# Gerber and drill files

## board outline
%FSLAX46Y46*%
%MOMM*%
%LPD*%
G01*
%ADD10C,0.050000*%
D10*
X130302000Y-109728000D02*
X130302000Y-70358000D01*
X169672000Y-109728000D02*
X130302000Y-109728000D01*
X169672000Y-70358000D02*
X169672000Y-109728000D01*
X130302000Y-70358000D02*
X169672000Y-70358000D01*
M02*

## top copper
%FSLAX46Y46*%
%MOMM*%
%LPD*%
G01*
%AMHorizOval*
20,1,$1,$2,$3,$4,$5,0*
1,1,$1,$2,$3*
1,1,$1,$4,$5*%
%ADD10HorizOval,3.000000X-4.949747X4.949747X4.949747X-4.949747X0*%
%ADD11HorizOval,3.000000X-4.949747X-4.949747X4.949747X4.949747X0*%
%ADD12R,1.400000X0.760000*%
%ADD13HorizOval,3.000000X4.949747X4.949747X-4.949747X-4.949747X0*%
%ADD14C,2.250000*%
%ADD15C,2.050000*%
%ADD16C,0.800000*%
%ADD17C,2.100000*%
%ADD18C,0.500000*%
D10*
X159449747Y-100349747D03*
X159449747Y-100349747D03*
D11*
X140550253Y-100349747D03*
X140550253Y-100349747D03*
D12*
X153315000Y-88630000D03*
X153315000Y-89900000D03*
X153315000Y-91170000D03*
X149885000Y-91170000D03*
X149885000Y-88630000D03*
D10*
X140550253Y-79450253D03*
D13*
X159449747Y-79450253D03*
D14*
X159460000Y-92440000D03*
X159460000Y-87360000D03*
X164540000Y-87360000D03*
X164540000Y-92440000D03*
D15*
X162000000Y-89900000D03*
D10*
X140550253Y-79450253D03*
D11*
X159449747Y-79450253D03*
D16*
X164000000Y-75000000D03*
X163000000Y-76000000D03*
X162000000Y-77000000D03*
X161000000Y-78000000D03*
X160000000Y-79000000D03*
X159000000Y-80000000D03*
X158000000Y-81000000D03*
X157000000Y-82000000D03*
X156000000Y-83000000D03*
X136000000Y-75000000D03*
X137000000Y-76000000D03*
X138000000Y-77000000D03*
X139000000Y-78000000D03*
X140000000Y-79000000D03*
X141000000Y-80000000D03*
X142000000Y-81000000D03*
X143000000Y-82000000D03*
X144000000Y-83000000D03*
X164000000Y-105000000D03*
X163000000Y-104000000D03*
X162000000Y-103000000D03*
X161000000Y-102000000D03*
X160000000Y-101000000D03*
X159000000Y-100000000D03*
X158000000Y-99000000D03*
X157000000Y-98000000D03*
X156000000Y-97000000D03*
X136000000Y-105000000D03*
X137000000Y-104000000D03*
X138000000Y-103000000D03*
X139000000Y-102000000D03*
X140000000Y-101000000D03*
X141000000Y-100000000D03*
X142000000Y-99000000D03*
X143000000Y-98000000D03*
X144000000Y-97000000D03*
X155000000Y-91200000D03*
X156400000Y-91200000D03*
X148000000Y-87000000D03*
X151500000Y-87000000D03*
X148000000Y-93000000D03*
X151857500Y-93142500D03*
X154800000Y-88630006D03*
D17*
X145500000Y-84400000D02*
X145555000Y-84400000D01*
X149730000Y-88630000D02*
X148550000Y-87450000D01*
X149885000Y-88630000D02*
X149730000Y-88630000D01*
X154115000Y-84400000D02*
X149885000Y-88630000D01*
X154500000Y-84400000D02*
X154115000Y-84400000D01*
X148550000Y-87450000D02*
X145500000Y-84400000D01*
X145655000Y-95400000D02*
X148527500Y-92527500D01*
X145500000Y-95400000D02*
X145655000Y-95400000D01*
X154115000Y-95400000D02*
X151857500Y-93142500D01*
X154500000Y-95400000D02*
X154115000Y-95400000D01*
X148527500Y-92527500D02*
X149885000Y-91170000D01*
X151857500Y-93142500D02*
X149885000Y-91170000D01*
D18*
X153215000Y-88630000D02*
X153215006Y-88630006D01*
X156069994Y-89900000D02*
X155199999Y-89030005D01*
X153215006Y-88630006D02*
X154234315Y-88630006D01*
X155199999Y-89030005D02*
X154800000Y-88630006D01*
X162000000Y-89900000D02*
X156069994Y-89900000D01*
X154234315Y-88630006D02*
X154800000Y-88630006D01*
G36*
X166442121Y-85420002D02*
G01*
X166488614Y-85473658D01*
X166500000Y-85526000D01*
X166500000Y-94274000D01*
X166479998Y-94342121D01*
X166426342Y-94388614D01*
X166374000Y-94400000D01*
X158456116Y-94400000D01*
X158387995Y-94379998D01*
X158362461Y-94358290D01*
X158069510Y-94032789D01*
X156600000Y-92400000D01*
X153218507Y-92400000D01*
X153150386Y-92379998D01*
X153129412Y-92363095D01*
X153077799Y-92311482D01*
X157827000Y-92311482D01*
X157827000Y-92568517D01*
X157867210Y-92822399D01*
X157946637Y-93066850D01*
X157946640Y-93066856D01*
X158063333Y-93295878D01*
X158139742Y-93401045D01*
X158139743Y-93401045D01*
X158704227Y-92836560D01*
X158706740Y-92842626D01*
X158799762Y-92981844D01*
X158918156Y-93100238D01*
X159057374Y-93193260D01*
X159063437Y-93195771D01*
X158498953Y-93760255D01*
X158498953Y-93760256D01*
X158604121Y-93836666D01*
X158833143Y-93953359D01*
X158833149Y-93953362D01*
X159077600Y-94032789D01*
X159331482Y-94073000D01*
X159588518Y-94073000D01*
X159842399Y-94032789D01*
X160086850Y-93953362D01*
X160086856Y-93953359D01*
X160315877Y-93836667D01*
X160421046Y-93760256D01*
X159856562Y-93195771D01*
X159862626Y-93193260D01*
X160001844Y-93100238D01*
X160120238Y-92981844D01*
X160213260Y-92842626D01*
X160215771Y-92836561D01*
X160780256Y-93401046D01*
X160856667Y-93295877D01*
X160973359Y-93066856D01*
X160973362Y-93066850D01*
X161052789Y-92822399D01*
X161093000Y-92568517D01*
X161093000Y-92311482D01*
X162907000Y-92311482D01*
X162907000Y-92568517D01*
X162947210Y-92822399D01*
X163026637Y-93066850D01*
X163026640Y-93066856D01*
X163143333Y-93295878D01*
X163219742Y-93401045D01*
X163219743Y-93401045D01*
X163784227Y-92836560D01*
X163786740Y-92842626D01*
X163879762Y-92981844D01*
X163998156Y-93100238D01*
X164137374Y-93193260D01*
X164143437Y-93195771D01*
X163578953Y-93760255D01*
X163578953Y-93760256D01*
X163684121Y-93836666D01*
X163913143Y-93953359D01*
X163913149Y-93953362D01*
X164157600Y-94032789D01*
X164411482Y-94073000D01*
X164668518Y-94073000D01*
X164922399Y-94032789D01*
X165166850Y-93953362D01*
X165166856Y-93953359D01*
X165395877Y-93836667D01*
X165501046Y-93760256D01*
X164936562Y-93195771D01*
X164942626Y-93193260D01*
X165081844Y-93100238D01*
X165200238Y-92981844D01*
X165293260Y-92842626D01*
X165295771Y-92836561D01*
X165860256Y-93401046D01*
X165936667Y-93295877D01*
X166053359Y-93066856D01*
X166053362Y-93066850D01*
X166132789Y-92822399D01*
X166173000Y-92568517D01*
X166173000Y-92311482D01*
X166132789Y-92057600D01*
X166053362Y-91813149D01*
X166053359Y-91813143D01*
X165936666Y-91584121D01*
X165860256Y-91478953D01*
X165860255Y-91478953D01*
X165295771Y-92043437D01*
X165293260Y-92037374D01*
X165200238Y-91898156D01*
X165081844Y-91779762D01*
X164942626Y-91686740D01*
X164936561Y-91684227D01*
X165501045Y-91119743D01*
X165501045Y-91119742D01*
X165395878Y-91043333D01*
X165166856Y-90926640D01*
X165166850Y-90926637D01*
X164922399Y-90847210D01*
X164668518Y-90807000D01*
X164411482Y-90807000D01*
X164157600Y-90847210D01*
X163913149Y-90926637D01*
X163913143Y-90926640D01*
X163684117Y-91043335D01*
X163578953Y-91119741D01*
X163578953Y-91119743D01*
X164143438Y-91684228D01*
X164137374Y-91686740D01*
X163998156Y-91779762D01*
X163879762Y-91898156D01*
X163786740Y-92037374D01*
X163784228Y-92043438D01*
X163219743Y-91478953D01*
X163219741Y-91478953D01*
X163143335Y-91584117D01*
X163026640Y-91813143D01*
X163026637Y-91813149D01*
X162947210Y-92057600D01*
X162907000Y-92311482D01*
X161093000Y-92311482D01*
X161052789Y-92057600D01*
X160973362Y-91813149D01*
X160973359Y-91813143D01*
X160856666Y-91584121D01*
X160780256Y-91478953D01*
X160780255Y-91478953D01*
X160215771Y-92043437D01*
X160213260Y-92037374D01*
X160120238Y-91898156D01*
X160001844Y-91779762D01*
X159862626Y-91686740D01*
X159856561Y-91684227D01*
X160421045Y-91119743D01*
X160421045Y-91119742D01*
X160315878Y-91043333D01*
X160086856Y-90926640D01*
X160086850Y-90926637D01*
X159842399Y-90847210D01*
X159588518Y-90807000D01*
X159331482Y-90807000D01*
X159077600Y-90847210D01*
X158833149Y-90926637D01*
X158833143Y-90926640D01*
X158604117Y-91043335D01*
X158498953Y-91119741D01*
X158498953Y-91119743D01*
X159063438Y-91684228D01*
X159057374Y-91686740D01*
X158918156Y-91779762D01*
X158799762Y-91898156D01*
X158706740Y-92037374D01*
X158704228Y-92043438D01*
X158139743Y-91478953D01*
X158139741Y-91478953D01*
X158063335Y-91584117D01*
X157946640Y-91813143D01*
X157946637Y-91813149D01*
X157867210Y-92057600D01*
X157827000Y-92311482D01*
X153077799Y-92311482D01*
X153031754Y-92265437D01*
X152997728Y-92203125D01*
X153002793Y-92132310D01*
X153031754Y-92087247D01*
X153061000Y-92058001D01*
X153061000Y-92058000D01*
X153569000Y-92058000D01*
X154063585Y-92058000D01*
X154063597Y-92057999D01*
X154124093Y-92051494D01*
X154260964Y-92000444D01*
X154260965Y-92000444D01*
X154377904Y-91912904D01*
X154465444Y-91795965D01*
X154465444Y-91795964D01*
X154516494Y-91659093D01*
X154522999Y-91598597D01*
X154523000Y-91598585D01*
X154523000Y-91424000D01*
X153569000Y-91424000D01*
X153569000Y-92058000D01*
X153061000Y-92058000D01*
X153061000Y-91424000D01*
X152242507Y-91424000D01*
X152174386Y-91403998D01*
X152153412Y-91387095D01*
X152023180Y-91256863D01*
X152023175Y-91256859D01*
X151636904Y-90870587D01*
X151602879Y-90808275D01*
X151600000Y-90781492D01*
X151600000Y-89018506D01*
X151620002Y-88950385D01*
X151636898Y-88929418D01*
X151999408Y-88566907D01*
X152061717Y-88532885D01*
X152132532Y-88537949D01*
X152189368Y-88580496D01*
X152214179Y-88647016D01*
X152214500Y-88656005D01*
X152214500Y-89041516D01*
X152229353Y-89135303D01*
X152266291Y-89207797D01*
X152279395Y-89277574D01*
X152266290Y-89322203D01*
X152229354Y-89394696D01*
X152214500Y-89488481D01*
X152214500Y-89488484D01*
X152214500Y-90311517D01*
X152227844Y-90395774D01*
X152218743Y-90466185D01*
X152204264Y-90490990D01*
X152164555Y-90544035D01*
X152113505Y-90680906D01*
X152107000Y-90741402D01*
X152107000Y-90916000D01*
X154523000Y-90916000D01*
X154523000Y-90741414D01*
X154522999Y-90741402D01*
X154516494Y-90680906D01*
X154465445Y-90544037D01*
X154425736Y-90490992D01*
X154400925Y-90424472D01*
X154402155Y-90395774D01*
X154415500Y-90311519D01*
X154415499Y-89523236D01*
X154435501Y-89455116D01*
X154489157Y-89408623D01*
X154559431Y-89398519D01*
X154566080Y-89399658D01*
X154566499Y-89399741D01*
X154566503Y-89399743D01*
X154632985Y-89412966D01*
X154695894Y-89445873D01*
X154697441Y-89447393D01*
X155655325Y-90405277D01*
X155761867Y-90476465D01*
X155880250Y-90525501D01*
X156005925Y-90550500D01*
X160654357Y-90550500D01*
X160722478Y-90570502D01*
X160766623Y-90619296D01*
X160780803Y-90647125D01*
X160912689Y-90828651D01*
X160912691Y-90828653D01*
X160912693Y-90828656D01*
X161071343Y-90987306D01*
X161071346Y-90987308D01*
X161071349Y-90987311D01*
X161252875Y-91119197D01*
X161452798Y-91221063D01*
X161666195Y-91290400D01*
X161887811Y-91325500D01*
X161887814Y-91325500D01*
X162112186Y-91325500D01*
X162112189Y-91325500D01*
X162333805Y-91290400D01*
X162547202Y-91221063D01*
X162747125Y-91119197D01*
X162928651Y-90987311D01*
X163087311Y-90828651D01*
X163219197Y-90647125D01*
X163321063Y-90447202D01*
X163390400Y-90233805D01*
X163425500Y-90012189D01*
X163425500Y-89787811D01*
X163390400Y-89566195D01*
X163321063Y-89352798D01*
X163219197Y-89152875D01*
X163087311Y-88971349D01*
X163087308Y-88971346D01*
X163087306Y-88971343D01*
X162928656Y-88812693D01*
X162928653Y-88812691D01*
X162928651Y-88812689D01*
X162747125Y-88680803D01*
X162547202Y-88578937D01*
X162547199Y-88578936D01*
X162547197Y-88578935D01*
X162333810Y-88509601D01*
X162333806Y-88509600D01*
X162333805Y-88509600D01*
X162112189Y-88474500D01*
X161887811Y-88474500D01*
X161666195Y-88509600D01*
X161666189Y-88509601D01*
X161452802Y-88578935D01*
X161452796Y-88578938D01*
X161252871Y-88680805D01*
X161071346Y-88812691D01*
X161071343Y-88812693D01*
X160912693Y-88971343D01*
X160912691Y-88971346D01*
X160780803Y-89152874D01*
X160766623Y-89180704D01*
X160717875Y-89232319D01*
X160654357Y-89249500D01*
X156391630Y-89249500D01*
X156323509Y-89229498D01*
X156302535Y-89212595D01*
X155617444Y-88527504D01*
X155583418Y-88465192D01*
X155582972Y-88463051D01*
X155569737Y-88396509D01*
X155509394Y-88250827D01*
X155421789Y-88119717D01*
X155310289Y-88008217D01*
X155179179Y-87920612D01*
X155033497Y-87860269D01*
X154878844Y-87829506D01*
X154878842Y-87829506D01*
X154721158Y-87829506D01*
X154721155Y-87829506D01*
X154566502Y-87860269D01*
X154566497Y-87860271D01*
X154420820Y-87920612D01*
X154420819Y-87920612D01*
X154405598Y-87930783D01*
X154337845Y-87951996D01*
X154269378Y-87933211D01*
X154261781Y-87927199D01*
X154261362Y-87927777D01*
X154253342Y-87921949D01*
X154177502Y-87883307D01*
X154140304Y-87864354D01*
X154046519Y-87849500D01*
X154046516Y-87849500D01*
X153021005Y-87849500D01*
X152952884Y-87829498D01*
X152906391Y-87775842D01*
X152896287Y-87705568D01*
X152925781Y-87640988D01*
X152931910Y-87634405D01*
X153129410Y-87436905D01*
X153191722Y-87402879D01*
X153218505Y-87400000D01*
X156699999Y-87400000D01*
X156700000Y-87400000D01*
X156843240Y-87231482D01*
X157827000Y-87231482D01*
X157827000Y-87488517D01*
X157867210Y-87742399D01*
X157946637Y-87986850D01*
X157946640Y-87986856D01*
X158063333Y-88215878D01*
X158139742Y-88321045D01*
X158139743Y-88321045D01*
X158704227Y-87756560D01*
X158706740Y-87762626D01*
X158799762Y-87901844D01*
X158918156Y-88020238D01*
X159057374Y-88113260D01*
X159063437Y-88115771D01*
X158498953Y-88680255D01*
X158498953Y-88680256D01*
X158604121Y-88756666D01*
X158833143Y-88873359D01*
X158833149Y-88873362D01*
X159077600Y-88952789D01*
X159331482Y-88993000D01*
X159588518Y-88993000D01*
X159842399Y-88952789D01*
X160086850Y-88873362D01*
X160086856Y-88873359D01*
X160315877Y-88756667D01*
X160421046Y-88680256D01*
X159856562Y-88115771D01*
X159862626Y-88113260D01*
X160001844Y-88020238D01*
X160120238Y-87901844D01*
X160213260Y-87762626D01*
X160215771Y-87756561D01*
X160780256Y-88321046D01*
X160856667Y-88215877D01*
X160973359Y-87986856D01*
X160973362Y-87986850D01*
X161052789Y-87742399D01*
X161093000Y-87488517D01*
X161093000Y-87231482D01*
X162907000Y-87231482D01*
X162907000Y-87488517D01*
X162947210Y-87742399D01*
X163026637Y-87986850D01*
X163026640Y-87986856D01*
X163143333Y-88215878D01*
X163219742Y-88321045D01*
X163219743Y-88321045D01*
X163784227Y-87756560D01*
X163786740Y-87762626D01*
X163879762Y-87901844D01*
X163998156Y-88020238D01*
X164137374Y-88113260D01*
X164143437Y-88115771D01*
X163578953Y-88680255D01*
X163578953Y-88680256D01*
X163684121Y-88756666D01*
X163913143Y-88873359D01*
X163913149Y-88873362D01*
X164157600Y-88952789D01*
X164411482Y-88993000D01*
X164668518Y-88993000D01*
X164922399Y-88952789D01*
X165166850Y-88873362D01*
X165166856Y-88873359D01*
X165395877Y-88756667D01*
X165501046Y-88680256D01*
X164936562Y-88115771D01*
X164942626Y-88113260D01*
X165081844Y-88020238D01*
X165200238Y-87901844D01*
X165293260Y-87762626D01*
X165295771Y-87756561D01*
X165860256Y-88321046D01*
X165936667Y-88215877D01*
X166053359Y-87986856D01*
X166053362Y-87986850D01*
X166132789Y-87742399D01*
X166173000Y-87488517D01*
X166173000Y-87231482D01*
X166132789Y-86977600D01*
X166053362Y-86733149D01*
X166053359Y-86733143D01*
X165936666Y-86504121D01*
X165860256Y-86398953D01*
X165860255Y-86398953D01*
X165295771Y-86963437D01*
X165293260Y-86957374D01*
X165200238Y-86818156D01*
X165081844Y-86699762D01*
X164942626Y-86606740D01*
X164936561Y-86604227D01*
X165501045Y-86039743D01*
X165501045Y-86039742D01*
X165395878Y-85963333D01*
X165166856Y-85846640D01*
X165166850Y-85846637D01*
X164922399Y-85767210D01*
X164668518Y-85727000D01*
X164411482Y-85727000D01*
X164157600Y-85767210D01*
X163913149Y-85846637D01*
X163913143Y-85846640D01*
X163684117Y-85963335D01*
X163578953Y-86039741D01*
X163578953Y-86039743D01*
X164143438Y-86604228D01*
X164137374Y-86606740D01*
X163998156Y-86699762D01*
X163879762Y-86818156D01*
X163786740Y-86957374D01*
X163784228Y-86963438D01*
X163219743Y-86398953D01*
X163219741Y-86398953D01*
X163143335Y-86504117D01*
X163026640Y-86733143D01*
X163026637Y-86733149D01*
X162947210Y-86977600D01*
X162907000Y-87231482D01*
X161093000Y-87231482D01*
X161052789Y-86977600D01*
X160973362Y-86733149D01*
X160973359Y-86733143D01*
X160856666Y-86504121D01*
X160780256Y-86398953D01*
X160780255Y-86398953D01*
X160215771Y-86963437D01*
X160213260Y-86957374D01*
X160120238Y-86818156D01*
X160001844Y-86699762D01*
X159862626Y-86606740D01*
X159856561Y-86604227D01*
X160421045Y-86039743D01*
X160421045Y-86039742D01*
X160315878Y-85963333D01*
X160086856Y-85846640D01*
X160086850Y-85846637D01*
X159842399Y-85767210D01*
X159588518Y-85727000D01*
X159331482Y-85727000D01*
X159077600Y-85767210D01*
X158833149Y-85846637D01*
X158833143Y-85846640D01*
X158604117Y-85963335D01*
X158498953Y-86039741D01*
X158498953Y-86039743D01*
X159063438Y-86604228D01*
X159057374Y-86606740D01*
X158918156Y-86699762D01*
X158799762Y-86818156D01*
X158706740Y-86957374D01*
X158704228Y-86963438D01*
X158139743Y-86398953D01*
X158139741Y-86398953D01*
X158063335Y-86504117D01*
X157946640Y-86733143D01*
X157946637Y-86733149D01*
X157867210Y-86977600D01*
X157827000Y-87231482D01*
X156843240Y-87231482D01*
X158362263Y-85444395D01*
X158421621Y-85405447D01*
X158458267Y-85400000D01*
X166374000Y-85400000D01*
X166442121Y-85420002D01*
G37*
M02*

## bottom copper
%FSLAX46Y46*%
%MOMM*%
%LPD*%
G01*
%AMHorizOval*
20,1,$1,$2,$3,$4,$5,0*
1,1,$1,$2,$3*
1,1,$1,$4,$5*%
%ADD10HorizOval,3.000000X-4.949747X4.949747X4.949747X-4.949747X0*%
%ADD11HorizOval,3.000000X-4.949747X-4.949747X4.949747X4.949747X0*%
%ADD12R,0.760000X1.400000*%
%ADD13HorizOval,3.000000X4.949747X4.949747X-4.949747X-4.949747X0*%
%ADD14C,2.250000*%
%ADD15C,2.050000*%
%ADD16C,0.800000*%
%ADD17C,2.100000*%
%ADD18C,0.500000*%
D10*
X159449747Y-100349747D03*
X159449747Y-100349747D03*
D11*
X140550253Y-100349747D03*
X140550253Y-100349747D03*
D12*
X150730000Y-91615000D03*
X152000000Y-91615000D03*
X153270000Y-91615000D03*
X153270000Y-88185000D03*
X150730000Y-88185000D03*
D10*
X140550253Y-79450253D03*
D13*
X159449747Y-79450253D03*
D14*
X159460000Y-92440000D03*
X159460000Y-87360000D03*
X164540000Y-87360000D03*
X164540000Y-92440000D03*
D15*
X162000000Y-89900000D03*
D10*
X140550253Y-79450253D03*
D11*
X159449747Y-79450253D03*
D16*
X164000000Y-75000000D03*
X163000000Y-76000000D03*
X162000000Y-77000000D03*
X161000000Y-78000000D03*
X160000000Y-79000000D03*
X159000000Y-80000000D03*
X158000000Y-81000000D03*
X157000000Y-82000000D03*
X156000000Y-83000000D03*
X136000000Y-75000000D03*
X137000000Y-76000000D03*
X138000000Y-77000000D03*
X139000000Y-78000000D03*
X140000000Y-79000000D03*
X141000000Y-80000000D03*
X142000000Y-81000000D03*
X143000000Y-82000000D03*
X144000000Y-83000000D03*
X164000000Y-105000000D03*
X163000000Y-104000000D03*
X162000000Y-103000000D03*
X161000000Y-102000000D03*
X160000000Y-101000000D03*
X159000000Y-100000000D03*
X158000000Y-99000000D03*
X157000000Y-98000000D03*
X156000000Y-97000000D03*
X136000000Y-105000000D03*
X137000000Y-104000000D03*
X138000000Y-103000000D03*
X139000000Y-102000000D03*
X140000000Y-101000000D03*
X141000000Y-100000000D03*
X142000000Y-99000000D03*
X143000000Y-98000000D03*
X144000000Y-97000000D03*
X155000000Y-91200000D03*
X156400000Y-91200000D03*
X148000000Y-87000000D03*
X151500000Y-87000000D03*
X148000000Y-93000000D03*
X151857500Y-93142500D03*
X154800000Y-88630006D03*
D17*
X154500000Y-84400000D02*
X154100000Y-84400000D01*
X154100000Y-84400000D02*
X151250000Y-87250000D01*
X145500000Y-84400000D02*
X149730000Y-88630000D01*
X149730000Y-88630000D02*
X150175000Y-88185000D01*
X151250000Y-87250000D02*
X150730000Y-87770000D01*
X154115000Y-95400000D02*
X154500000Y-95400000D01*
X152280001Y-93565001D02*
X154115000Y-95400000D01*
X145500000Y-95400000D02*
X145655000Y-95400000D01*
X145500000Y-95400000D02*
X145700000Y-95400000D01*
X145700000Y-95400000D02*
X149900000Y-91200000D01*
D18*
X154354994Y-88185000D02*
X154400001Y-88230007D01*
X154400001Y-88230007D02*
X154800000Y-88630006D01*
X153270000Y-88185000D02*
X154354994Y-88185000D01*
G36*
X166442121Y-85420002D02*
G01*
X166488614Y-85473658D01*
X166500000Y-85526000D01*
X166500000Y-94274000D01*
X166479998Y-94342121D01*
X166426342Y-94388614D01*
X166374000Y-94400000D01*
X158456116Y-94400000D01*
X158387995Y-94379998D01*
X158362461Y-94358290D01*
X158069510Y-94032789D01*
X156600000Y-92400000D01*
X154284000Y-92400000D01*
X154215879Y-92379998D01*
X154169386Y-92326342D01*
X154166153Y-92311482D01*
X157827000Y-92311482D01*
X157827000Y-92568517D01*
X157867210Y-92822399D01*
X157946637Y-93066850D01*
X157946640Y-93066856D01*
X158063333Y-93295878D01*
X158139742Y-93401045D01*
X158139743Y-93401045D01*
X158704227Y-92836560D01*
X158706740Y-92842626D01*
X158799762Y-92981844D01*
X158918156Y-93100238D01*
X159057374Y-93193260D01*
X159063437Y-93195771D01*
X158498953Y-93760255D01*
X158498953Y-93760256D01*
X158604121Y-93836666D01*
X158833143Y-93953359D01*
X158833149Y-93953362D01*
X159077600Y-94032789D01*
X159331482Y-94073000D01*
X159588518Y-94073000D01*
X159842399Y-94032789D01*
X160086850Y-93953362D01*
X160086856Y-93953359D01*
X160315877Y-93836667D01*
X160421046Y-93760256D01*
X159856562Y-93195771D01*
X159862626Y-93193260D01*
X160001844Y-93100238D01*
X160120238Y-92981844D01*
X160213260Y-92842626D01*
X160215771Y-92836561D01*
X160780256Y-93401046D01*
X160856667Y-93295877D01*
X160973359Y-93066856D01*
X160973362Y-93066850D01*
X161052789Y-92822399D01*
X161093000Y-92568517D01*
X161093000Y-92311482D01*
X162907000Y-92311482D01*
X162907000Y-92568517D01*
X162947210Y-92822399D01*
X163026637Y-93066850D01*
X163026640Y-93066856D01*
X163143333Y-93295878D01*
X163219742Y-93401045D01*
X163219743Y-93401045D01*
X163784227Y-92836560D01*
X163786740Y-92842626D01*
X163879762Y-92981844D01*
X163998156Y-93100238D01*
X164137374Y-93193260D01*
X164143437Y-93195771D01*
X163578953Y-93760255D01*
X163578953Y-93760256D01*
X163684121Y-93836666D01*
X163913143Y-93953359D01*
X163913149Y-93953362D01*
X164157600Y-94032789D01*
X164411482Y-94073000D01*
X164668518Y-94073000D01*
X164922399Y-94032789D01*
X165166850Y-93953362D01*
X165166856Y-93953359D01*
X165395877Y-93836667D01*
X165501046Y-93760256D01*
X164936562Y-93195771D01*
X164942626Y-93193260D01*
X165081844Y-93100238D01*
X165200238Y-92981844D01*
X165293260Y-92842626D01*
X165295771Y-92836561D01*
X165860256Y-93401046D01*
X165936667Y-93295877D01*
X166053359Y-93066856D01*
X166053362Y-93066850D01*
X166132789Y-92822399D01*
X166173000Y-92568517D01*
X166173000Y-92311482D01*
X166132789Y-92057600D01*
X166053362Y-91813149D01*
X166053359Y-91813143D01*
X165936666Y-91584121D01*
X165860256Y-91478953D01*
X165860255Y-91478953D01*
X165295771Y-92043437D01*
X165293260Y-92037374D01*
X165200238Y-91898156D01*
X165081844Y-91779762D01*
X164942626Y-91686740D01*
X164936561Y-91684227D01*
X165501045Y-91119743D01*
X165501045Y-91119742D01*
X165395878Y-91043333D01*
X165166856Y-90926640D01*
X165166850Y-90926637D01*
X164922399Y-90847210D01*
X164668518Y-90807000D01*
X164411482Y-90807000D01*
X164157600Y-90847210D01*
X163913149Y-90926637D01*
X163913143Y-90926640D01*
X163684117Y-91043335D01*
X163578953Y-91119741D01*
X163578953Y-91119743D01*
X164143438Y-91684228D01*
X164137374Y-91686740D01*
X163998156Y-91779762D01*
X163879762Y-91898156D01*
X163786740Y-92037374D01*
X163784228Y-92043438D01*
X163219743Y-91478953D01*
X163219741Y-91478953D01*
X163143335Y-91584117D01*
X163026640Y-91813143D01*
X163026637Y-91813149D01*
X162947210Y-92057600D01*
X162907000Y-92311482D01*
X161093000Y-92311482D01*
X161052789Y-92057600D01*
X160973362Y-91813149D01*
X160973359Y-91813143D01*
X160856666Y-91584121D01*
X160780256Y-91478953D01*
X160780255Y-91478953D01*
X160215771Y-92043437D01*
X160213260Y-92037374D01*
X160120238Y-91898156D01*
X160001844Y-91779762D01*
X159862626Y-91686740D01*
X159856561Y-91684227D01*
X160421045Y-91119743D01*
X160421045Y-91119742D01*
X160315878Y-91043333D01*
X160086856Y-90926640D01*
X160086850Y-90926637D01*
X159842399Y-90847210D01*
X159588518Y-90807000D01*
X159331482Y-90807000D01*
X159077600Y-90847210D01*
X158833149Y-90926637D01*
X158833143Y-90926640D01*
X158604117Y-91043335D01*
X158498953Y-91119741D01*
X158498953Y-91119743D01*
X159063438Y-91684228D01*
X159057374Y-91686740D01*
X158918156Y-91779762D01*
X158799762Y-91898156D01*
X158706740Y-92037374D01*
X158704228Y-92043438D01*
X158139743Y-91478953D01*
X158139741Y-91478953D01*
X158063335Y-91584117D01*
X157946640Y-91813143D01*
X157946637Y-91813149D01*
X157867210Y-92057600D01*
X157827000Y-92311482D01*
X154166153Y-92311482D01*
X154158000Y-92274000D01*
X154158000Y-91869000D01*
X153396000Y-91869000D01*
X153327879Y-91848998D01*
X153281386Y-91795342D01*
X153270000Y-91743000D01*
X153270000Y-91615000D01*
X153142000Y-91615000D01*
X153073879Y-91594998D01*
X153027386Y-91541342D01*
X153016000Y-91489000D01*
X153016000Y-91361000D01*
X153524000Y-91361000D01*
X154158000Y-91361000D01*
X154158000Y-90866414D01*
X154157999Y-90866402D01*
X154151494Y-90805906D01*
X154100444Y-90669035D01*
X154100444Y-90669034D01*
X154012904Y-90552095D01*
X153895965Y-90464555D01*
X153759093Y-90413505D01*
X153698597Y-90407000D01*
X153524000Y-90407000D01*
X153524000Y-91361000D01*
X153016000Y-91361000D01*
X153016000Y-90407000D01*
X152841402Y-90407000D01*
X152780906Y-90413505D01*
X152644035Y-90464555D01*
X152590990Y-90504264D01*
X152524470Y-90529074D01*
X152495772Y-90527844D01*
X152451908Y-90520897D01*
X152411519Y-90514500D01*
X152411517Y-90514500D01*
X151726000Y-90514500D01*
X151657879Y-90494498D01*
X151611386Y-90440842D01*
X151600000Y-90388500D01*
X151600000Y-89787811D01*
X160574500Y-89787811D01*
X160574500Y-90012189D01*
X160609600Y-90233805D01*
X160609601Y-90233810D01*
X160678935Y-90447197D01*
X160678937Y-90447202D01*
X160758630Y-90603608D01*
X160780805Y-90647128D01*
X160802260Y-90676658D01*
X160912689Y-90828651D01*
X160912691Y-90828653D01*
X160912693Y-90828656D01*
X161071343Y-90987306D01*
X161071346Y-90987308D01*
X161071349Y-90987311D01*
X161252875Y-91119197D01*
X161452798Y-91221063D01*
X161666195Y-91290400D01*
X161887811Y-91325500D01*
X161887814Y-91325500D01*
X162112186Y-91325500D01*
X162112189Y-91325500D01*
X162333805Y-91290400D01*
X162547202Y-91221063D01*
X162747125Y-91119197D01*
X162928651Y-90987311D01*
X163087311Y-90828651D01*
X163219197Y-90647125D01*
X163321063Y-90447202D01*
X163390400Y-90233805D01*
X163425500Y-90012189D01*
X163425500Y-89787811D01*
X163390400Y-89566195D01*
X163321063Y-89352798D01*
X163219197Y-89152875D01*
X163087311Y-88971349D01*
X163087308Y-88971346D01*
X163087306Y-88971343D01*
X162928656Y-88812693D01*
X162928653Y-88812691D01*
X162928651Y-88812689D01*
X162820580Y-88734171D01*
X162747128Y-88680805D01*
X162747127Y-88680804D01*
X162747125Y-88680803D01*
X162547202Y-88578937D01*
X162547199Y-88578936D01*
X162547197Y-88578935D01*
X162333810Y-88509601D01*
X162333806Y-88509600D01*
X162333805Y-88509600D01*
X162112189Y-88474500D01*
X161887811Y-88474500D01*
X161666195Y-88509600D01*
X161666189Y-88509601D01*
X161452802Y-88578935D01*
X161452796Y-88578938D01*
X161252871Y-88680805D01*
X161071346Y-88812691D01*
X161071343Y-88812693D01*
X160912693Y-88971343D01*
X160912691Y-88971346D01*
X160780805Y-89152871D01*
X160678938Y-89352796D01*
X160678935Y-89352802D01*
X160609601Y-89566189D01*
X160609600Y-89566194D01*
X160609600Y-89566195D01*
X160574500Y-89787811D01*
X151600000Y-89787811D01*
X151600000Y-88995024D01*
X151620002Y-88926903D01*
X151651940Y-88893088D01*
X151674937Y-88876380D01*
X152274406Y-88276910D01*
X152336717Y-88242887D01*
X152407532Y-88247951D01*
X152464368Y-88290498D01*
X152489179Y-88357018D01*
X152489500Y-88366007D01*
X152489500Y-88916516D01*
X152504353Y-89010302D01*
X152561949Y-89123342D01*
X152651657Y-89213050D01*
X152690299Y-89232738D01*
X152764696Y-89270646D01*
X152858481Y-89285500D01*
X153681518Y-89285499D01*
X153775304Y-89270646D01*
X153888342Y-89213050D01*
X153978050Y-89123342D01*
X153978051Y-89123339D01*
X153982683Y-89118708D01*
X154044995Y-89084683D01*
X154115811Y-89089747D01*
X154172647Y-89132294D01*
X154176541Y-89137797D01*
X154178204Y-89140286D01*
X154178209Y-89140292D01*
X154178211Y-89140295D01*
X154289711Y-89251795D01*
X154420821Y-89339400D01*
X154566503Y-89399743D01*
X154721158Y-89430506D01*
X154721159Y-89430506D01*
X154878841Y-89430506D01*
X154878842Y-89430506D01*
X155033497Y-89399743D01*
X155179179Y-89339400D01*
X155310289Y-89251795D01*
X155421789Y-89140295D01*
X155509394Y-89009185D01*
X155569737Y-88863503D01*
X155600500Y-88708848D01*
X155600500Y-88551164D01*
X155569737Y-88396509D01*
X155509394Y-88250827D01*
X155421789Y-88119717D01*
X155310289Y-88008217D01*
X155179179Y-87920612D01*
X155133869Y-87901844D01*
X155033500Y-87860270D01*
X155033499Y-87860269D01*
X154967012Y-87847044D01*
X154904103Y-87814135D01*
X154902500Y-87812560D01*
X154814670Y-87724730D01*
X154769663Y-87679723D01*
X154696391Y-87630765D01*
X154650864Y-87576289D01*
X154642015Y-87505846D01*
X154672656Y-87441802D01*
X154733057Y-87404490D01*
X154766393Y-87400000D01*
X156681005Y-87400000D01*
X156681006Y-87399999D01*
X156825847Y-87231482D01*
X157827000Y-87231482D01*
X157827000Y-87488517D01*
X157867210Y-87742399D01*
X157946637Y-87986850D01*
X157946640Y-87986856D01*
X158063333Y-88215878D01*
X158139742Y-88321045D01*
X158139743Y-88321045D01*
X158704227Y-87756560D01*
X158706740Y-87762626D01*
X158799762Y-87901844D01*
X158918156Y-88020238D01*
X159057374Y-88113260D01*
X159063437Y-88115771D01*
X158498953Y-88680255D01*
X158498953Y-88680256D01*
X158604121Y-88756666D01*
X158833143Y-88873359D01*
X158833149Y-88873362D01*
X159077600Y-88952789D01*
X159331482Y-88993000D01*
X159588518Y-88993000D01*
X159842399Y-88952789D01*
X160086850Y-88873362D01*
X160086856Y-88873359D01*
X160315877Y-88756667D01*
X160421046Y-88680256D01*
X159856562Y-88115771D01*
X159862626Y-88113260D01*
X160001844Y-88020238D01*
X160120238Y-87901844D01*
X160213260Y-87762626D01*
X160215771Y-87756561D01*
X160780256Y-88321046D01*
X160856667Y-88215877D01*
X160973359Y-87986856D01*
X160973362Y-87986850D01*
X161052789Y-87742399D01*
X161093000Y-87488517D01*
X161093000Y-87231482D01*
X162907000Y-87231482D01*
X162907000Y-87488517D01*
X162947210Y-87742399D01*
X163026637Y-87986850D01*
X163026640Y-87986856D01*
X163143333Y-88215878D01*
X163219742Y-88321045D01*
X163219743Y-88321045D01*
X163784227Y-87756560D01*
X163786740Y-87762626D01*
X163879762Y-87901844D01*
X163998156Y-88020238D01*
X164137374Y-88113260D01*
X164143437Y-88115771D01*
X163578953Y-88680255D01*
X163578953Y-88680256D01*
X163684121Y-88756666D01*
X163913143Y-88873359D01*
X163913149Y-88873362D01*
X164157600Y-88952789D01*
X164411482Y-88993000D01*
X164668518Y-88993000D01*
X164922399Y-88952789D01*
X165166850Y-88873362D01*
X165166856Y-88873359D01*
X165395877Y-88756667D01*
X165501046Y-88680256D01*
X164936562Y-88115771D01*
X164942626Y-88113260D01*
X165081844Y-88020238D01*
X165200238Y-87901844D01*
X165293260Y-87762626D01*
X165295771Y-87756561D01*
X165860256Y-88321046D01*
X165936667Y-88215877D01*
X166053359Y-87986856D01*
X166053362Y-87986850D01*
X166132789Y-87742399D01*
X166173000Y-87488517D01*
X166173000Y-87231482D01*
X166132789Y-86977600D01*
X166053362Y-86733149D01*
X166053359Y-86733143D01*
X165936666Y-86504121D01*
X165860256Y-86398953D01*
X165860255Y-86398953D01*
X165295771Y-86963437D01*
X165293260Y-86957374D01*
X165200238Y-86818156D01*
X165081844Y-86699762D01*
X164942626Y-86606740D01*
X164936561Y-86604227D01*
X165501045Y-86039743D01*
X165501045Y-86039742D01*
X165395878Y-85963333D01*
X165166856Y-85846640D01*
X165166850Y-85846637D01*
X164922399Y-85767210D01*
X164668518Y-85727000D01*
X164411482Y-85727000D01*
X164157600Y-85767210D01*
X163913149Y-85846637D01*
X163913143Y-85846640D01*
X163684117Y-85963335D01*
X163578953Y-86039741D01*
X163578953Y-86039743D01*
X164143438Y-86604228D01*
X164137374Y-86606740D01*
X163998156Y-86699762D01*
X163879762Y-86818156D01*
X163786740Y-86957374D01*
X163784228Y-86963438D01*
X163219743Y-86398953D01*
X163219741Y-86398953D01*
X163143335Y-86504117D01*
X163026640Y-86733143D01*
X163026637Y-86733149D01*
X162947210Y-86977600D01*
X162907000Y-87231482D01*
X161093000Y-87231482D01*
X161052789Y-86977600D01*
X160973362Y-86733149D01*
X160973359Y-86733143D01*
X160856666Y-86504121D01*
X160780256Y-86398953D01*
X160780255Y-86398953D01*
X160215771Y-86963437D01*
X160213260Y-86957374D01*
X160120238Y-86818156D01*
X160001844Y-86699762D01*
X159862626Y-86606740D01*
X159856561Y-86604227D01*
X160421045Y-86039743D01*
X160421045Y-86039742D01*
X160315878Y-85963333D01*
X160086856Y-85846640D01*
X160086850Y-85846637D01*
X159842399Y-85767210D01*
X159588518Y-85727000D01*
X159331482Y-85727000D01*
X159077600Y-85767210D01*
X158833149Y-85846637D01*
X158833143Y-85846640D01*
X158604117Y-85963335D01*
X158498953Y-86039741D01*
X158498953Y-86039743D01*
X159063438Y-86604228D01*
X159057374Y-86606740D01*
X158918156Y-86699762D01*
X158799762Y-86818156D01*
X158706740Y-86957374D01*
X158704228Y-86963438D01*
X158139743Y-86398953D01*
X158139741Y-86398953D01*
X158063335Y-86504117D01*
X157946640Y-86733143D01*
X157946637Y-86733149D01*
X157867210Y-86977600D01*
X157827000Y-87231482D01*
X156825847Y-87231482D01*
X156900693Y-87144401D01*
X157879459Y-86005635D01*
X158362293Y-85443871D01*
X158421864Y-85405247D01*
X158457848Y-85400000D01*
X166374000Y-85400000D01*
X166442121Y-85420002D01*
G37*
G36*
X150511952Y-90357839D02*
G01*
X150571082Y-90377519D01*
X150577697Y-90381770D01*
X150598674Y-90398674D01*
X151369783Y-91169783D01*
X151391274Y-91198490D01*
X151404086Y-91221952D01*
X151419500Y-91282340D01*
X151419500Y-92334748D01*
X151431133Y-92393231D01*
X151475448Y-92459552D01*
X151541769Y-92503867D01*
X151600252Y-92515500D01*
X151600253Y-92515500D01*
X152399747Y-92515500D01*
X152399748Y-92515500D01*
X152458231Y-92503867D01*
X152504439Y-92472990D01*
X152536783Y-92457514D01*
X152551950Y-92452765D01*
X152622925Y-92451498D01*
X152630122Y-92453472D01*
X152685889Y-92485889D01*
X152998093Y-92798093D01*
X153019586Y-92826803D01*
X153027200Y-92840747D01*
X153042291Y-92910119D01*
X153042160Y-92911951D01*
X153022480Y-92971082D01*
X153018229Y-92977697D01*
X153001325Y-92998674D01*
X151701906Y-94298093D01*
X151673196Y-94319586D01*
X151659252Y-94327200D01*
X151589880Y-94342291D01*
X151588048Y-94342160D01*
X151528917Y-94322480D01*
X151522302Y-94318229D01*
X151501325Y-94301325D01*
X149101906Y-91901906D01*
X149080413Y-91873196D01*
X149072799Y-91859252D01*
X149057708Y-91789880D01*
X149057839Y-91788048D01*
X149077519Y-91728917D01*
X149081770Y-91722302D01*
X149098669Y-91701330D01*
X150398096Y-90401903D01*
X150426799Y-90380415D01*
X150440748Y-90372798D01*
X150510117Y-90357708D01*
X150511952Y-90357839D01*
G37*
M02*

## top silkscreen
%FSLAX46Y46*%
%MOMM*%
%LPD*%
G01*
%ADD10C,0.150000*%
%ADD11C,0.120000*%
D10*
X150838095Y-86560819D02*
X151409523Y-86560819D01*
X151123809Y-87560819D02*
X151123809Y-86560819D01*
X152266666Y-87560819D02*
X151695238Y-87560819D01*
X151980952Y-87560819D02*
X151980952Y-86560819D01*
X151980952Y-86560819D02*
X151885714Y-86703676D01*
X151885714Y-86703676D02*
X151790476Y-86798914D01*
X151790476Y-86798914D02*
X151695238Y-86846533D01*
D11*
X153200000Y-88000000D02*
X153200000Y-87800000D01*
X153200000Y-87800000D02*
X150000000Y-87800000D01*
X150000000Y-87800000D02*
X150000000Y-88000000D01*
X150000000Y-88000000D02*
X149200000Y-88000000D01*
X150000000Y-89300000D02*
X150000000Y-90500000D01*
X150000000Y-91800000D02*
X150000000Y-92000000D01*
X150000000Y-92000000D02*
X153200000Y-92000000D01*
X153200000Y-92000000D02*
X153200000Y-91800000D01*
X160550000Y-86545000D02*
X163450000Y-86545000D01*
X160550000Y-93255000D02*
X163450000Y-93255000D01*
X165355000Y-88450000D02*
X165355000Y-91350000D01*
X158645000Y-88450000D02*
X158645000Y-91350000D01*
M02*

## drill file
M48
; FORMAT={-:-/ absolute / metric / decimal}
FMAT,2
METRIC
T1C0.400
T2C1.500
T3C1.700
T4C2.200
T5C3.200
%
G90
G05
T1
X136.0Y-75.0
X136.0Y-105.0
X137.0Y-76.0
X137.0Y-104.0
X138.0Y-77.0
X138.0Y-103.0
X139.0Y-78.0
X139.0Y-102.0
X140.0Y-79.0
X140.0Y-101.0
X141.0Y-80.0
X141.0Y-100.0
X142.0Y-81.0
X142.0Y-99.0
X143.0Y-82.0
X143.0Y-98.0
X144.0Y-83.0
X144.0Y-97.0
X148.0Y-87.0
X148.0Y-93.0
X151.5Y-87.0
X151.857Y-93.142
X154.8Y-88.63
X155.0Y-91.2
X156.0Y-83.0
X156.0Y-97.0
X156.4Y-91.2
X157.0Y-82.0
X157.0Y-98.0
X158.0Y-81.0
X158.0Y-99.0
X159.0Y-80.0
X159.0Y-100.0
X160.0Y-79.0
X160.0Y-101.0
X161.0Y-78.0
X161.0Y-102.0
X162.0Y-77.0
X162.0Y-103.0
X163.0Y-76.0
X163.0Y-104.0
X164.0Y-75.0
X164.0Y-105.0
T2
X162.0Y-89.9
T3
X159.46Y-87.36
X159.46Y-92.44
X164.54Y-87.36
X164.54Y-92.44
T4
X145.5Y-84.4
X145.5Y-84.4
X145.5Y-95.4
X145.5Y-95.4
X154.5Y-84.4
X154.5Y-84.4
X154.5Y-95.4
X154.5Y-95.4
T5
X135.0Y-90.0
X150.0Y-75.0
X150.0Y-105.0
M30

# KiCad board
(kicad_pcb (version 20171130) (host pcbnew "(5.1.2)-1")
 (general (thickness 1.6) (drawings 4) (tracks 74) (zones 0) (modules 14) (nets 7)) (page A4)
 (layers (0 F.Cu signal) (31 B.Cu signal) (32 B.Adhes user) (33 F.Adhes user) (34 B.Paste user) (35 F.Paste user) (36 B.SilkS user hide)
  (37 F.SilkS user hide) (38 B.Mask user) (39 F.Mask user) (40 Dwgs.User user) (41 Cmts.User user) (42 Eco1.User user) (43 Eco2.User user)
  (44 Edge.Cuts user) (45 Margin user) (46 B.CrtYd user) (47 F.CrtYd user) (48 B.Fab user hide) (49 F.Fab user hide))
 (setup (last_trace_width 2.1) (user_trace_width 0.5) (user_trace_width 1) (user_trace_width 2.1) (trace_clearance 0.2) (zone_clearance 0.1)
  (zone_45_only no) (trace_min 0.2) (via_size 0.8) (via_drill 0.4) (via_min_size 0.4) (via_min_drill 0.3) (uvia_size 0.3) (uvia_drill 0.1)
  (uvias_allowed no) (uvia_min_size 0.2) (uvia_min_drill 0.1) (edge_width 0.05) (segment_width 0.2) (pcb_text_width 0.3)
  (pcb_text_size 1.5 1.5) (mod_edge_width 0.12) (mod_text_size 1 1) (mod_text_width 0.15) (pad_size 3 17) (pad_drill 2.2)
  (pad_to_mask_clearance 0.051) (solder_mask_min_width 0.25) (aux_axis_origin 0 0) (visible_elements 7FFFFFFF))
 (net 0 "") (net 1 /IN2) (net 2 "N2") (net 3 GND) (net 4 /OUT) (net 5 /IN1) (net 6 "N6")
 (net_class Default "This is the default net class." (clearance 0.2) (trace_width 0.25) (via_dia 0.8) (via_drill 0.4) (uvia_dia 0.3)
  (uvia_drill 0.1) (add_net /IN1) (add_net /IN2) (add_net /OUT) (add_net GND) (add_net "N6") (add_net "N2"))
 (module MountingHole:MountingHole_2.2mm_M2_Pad (layer B.Cu) (at 154.5 95.4 90)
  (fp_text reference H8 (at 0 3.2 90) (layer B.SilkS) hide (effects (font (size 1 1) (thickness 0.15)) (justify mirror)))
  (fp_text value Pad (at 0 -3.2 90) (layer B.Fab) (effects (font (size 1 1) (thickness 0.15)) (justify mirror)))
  (pad 1 thru_hole oval (at 0 0 45) (size 3 17) (drill 2.2 (offset 0 7)) (layers *.Cu *.Mask) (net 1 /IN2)))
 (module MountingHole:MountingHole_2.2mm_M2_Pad (layer F.Cu) (at 154.5 95.4 180)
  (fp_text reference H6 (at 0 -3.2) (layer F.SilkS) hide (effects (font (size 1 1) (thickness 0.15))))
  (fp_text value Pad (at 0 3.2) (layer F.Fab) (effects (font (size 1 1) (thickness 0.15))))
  (pad 1 thru_hole oval (at 0 0 225) (size 3 17) (drill 2.2 (offset 0 -7)) (layers *.Cu *.Mask) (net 1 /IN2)))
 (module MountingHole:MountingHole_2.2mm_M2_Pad (layer B.Cu) (at 145.5 95.4)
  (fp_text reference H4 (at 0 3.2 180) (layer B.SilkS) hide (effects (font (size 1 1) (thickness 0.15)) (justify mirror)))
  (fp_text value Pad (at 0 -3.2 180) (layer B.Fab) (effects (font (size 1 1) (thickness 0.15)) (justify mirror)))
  (pad 1 thru_hole oval (at 0 0 315) (size 3 17) (drill 2.2 (offset 0 7)) (layers *.Cu *.Mask) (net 1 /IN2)))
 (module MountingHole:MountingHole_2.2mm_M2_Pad (layer B.Cu) (at 145.5 95.4)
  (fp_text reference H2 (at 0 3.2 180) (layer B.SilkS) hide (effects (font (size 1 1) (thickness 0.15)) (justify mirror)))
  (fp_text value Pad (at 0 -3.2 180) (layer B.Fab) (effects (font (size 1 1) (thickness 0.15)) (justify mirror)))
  (pad 1 thru_hole oval (at 0 0 315) (size 3 17) (drill 2.2 (offset 0 7)) (layers *.Cu *.Mask) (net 1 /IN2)))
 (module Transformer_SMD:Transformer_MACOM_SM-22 (layer B.Cu) (at 152 89.9 270)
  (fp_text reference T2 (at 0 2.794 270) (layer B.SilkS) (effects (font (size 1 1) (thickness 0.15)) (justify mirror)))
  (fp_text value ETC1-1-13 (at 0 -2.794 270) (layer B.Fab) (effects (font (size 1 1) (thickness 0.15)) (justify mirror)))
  (pad 5 smd rect (at 1.715 1.27 270) (size 1.4 0.76) (layers B.Cu B.Paste B.Mask) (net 1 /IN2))
  (pad 4 smd rect (at 1.715 0 270) (size 1.4 0.76) (layers B.Cu B.Paste B.Mask) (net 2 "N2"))
  (pad 3 smd rect (at 1.715 -1.27 270) (size 1.4 0.76) (layers B.Cu B.Paste B.Mask) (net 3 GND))
  (pad 2 smd rect (at -1.715 -1.27 270) (size 1.4 0.76) (layers B.Cu B.Paste B.Mask) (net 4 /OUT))
  (pad 1 smd rect (at -1.715 1.27 270) (size 1.4 0.76) (layers B.Cu B.Paste B.Mask) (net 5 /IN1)))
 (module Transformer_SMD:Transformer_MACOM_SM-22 (layer F.Cu) (at 151.6 89.9)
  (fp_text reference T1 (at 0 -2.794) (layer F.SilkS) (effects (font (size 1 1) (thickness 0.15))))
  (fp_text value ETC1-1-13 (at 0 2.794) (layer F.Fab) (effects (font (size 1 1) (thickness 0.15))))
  (fp_line (start 1.6 -1.9) (end 1.6 -2.1) (layer F.SilkS) (width 0.12))
  (fp_line (start 1.6 -2.1) (end -1.6 -2.1) (layer F.SilkS) (width 0.12))
  (fp_line (start -1.6 -2.1) (end -1.6 -1.9) (layer F.SilkS) (width 0.12))
  (fp_line (start -1.6 -1.9) (end -2.4 -1.9) (layer F.SilkS) (width 0.12))
  (fp_line (start -1.6 -0.6) (end -1.6 0.6) (layer F.SilkS) (width 0.12))
  (fp_line (start -1.6 1.9) (end -1.6 2.1) (layer F.SilkS) (width 0.12))
  (fp_line (start -1.6 2.1) (end 1.6 2.1) (layer F.SilkS) (width 0.12))
  (fp_line (start 1.6 2.1) (end 1.6 1.9) (layer F.SilkS) (width 0.12))
  (pad 5 smd rect (at 1.715 -1.27) (size 1.4 0.76) (layers F.Cu F.Paste F.Mask) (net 4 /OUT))
  (pad 4 smd rect (at 1.715 0) (size 1.4 0.76) (layers F.Cu F.Paste F.Mask) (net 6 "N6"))
  (pad 3 smd rect (at 1.715 1.27) (size 1.4 0.76) (layers F.Cu F.Paste F.Mask) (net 3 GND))
  (pad 2 smd rect (at -1.715 1.27) (size 1.4 0.76) (layers F.Cu F.Paste F.Mask) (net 1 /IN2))
  (pad 1 smd rect (at -1.715 -1.27) (size 1.4 0.76) (layers F.Cu F.Paste F.Mask) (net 5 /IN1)))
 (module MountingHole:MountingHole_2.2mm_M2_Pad (layer B.Cu) (at 145.5 84.4 270)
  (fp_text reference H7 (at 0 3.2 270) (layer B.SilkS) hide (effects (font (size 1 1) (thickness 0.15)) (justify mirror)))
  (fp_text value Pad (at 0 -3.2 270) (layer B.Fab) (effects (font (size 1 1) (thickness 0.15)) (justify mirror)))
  (pad 1 thru_hole oval (at 0 0 225) (size 3 17) (drill 2.2 (offset 0 7)) (layers *.Cu *.Mask) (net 5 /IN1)))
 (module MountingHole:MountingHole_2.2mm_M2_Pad (layer B.Cu) (at 154.5 84.4 180)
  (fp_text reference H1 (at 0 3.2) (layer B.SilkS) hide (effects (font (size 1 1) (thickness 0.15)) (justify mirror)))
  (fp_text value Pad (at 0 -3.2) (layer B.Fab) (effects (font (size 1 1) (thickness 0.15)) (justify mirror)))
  (pad 1 thru_hole oval (at 0 0 135) (size 3 17) (drill 2.2 (offset 0 7)) (layers *.Cu *.Mask) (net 5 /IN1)))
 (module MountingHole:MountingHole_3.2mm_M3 (layer F.Cu) (at 150 105)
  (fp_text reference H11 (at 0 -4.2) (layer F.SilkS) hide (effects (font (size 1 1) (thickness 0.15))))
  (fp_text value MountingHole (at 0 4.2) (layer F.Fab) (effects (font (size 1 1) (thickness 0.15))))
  (pad 1 np_thru_hole circle (at 0 0) (size 3.2 3.2) (drill 3.2) (layers *.Cu *.Mask)))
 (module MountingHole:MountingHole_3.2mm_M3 (layer F.Cu) (at 150 75)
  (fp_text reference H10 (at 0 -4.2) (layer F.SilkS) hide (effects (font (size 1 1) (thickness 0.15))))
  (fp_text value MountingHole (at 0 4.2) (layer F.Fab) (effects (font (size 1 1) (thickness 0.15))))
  (pad 1 np_thru_hole circle (at 0 0) (size 3.2 3.2) (drill 3.2) (layers *.Cu *.Mask)))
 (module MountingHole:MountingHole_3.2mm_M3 (layer F.Cu) (at 135 90)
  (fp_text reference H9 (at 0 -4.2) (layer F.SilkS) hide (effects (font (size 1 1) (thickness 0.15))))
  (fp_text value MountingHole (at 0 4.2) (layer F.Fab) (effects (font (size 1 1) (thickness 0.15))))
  (pad 1 np_thru_hole circle (at 0 0) (size 3.2 3.2) (drill 3.2) (layers *.Cu *.Mask)))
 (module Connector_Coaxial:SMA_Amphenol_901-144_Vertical (layer F.Cu) (at 162 89.9)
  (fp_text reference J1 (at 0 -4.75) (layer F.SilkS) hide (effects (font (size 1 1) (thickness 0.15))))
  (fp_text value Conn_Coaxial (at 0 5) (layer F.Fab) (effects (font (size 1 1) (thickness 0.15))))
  (fp_line (start -1.45 -3.355) (end 1.45 -3.355) (layer F.SilkS) (width 0.12))
  (fp_line (start -1.45 3.355) (end 1.45 3.355) (layer F.SilkS) (width 0.12))
  (fp_line (start 3.355 -1.45) (end 3.355 1.45) (layer F.SilkS) (width 0.12))
  (fp_line (start -3.355 -1.45) (end -3.355 1.45) (layer F.SilkS) (width 0.12))
  (pad 2 thru_hole circle (at -2.54 2.54) (size 2.25 2.25) (drill 1.7) (layers *.Cu *.Mask) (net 3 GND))
  (pad 2 thru_hole circle (at -2.54 -2.54) (size 2.25 2.25) (drill 1.7) (layers *.Cu *.Mask) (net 3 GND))
  (pad 2 thru_hole circle (at 2.54 -2.54) (size 2.25 2.25) (drill 1.7) (layers *.Cu *.Mask) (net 3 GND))
  (pad 2 thru_hole circle (at 2.54 2.54) (size 2.25 2.25) (drill 1.7) (layers *.Cu *.Mask) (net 3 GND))
  (pad 1 thru_hole circle (at 0 0) (size 2.05 2.05) (drill 1.5) (layers *.Cu *.Mask) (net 4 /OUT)))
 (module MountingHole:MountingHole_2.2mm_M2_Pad (layer F.Cu) (at 145.5 84.4)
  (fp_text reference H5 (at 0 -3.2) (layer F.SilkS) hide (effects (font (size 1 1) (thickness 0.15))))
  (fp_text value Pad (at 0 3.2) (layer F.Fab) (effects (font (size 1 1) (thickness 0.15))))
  (pad 1 thru_hole oval (at 0 0 45) (size 3 17) (drill 2.2 (offset 0 -7)) (layers *.Cu *.Mask) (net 5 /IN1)))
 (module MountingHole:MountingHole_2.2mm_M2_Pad (layer F.Cu) (at 154.5 84.4 270)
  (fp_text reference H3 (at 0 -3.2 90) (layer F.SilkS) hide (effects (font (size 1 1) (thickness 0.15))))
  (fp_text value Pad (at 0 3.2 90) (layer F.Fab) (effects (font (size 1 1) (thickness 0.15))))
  (pad 1 thru_hole oval (at 0 0 315) (size 3 17) (drill 2.2 (offset 0 -7)) (layers *.Cu *.Mask) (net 5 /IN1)))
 (gr_line (start 130.302 109.728) (end 130.302 70.358) (layer Edge.Cuts) (width 0.05))
 (gr_line (start 169.672 109.728) (end 130.302 109.728) (layer Edge.Cuts) (width 0.05))
 (gr_line (start 169.672 70.358) (end 169.672 109.728) (layer Edge.Cuts) (width 0.05))
 (gr_line (start 130.302 70.358) (end 169.672 70.358) (layer Edge.Cuts) (width 0.05))
 (via (at 164 75) (size 0.8) (drill 0.4) (layers F.Cu B.Cu) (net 5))
 (via (at 163 76) (size 0.8) (drill 0.4) (layers F.Cu B.Cu) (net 5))
 (via (at 162 77) (size 0.8) (drill 0.4) (layers F.Cu B.Cu) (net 5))
 (via (at 161 78) (size 0.8) (drill 0.4) (layers F.Cu B.Cu) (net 5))
 (via (at 160 79) (size 0.8) (drill 0.4) (layers F.Cu B.Cu) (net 5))
 (via (at 159 80) (size 0.8) (drill 0.4) (layers F.Cu B.Cu) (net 5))
 (via (at 158 81) (size 0.8) (drill 0.4) (layers F.Cu B.Cu) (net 5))
 (via (at 157 82) (size 0.8) (drill 0.4) (layers F.Cu B.Cu) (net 5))
 (via (at 156 83) (size 0.8) (drill 0.4) (layers F.Cu B.Cu) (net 5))
 (via (at 136 75) (size 0.8) (drill 0.4) (layers F.Cu B.Cu) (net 5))
 (via (at 137 76) (size 0.8) (drill 0.4) (layers F.Cu B.Cu) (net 5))
 (via (at 138 77) (size 0.8) (drill 0.4) (layers F.Cu B.Cu) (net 5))
 (via (at 139 78) (size 0.8) (drill 0.4) (layers F.Cu B.Cu) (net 5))
 (via (at 140 79) (size 0.8) (drill 0.4) (layers F.Cu B.Cu) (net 5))
 (via (at 141 80) (size 0.8) (drill 0.4) (layers F.Cu B.Cu) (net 5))
 (via (at 142 81) (size 0.8) (drill 0.4) (layers F.Cu B.Cu) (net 5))
 (via (at 143 82) (size 0.8) (drill 0.4) (layers F.Cu B.Cu) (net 5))
 (via (at 144 83) (size 0.8) (drill 0.4) (layers F.Cu B.Cu) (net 5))
 (segment (start 145.5 84.4) (end 145.555 84.4) (width 2.1) (layer F.Cu) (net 5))
 (via (at 164 105) (size 0.8) (drill 0.4) (layers F.Cu B.Cu) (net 1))
 (via (at 163 104) (size 0.8) (drill 0.4) (layers F.Cu B.Cu) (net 1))
 (via (at 162 103) (size 0.8) (drill 0.4) (layers F.Cu B.Cu) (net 1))
 (via (at 161 102) (size 0.8) (drill 0.4) (layers F.Cu B.Cu) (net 1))
 (via (at 160 101) (size 0.8) (drill 0.4) (layers F.Cu B.Cu) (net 1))
 (via (at 159 100) (size 0.8) (drill 0.4) (layers F.Cu B.Cu) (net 1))
 (via (at 158 99) (size 0.8) (drill 0.4) (layers F.Cu B.Cu) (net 1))
 (via (at 157 98) (size 0.8) (drill 0.4) (layers F.Cu B.Cu) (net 1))
 (via (at 156 97) (size 0.8) (drill 0.4) (layers F.Cu B.Cu) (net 1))
 (via (at 136 105) (size 0.8) (drill 0.4) (layers F.Cu B.Cu) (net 1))
 (via (at 137 104) (size 0.8) (drill 0.4) (layers F.Cu B.Cu) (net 1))
 (via (at 138 103) (size 0.8) (drill 0.4) (layers F.Cu B.Cu) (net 1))
 (via (at 139 102) (size 0.8) (drill 0.4) (layers F.Cu B.Cu) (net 1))
 (via (at 140 101) (size 0.8) (drill 0.4) (layers F.Cu B.Cu) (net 1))
 (via (at 141 100) (size 0.8) (drill 0.4) (layers F.Cu B.Cu) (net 1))
 (via (at 142 99) (size 0.8) (drill 0.4) (layers F.Cu B.Cu) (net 1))
 (via (at 143 98) (size 0.8) (drill 0.4) (layers F.Cu B.Cu) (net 1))
 (via (at 144 97) (size 0.8) (drill 0.4) (layers F.Cu B.Cu) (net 1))
 (via (at 155 91.2) (size 0.8) (drill 0.4) (layers F.Cu B.Cu) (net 3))
 (via (at 156.4 91.2) (size 0.8) (drill 0.4) (layers F.Cu B.Cu) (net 3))
 (segment (start 149.73 88.63) (end 148.55 87.45) (width 2.1) (layer F.Cu) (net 5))
 (segment (start 149.885 88.63) (end 149.73 88.63) (width 2.1) (layer F.Cu) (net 5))
 (segment (start 154.115 84.4) (end 149.885 88.63) (width 2.1) (layer F.Cu) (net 5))
 (segment (start 154.5 84.4) (end 154.115 84.4) (width 2.1) (layer F.Cu) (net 5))
 (segment (start 154.5 84.4) (end 154.1 84.4) (width 2.1) (layer B.Cu) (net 5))
 (segment (start 154.1 84.4) (end 151.25 87.25) (width 2.1) (layer B.Cu) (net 5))
 (segment (start 145.5 84.4) (end 149.73 88.63) (width 2.1) (layer B.Cu) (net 5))
 (segment (start 149.73 88.63) (end 150.175 88.185) (width 2.1) (layer B.Cu) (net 5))
 (segment (start 148.55 87.45) (end 145.5 84.4) (width 2.1) (layer F.Cu) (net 5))
 (via (at 148 87) (size 0.8) (drill 0.4) (layers F.Cu B.Cu) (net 5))
 (segment (start 151.25 87.25) (end 150.73 87.77) (width 2.1) (layer B.Cu) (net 5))
 (via (at 151.5 87) (size 0.8) (drill 0.4) (layers F.Cu B.Cu) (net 5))
 (segment (start 145.655 95.4) (end 148.5275 92.5275) (width 2.1) (layer F.Cu) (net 1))
 (segment (start 145.5 95.4) (end 145.655 95.4) (width 2.1) (layer F.Cu) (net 1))
 (segment (start 154.115 95.4) (end 151.8575 93.1425) (width 2.1) (layer F.Cu) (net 1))
 (segment (start 154.5 95.4) (end 154.115 95.4) (width 2.1) (layer F.Cu) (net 1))
 (segment (start 154.115 95.4) (end 154.5 95.4) (width 2.1) (layer B.Cu) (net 1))
 (segment (start 152.280001 93.565001) (end 154.115 95.4) (width 2.1) (layer B.Cu) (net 1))
 (segment (start 145.5 95.4) (end 145.655 95.4) (width 2.1) (layer B.Cu) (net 1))
 (segment (start 145.5 95.4) (end 145.7 95.4) (width 2.1) (layer B.Cu) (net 1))
 (segment (start 145.7 95.4) (end 149.9 91.2) (width 2.1) (layer B.Cu) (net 1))
 (segment (start 148.5275 92.5275) (end 149.885 91.17) (width 2.1) (layer F.Cu) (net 1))
 (via (at 148 93) (size 0.8) (drill 0.4) (layers F.Cu B.Cu) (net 1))
 (segment (start 151.8575 93.1425) (end 149.885 91.17) (width 2.1) (layer F.Cu) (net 1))
 (via (at 151.8575 93.1425) (size 0.8) (drill 0.4) (layers F.Cu B.Cu) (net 1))
 (via (at 154.8 88.630006) (size 0.8) (drill 0.4) (layers F.Cu B.Cu) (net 4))
 (segment (start 153.215 88.63) (end 153.215006 88.630006) (width 0.5) (layer F.Cu) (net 4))
 (segment (start 156.069994 89.9) (end 155.199999 89.030005) (width 0.5) (layer F.Cu) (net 4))
 (segment (start 153.215006 88.630006) (end 154.234315 88.630006) (width 0.5) (layer F.Cu) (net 4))
 (segment (start 154.354994 88.185) (end 154.400001 88.230007) (width 0.5) (layer B.Cu) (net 4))
 (segment (start 154.400001 88.230007) (end 154.8 88.630006) (width 0.5) (layer B.Cu) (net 4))
 (segment (start 153.27 88.185) (end 154.354994 88.185) (width 0.5) (layer B.Cu) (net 4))
 (segment (start 155.199999 89.030005) (end 154.8 88.630006) (width 0.5) (layer F.Cu) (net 4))
 (segment (start 162 89.9) (end 156.069994 89.9) (width 0.5) (layer F.Cu) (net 4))
 (segment (start 154.234315 88.630006) (end 154.8 88.630006) (width 0.5) (layer F.Cu) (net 4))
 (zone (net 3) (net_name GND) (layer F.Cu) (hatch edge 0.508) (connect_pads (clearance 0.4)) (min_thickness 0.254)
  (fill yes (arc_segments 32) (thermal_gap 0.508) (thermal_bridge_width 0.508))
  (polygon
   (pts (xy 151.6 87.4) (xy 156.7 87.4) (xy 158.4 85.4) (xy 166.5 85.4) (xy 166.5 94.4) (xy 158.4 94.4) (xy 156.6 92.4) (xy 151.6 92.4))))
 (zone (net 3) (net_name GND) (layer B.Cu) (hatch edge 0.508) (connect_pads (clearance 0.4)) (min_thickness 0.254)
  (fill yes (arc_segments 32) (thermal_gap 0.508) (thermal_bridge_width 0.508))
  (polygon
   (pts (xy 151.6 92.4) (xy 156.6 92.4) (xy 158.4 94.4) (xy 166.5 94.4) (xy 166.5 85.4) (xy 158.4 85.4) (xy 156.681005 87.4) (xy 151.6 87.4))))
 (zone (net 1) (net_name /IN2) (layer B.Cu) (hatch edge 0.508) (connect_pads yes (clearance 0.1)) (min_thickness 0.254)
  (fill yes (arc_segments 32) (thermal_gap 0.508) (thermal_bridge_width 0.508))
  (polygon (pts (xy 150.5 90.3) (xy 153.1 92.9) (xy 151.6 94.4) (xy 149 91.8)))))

